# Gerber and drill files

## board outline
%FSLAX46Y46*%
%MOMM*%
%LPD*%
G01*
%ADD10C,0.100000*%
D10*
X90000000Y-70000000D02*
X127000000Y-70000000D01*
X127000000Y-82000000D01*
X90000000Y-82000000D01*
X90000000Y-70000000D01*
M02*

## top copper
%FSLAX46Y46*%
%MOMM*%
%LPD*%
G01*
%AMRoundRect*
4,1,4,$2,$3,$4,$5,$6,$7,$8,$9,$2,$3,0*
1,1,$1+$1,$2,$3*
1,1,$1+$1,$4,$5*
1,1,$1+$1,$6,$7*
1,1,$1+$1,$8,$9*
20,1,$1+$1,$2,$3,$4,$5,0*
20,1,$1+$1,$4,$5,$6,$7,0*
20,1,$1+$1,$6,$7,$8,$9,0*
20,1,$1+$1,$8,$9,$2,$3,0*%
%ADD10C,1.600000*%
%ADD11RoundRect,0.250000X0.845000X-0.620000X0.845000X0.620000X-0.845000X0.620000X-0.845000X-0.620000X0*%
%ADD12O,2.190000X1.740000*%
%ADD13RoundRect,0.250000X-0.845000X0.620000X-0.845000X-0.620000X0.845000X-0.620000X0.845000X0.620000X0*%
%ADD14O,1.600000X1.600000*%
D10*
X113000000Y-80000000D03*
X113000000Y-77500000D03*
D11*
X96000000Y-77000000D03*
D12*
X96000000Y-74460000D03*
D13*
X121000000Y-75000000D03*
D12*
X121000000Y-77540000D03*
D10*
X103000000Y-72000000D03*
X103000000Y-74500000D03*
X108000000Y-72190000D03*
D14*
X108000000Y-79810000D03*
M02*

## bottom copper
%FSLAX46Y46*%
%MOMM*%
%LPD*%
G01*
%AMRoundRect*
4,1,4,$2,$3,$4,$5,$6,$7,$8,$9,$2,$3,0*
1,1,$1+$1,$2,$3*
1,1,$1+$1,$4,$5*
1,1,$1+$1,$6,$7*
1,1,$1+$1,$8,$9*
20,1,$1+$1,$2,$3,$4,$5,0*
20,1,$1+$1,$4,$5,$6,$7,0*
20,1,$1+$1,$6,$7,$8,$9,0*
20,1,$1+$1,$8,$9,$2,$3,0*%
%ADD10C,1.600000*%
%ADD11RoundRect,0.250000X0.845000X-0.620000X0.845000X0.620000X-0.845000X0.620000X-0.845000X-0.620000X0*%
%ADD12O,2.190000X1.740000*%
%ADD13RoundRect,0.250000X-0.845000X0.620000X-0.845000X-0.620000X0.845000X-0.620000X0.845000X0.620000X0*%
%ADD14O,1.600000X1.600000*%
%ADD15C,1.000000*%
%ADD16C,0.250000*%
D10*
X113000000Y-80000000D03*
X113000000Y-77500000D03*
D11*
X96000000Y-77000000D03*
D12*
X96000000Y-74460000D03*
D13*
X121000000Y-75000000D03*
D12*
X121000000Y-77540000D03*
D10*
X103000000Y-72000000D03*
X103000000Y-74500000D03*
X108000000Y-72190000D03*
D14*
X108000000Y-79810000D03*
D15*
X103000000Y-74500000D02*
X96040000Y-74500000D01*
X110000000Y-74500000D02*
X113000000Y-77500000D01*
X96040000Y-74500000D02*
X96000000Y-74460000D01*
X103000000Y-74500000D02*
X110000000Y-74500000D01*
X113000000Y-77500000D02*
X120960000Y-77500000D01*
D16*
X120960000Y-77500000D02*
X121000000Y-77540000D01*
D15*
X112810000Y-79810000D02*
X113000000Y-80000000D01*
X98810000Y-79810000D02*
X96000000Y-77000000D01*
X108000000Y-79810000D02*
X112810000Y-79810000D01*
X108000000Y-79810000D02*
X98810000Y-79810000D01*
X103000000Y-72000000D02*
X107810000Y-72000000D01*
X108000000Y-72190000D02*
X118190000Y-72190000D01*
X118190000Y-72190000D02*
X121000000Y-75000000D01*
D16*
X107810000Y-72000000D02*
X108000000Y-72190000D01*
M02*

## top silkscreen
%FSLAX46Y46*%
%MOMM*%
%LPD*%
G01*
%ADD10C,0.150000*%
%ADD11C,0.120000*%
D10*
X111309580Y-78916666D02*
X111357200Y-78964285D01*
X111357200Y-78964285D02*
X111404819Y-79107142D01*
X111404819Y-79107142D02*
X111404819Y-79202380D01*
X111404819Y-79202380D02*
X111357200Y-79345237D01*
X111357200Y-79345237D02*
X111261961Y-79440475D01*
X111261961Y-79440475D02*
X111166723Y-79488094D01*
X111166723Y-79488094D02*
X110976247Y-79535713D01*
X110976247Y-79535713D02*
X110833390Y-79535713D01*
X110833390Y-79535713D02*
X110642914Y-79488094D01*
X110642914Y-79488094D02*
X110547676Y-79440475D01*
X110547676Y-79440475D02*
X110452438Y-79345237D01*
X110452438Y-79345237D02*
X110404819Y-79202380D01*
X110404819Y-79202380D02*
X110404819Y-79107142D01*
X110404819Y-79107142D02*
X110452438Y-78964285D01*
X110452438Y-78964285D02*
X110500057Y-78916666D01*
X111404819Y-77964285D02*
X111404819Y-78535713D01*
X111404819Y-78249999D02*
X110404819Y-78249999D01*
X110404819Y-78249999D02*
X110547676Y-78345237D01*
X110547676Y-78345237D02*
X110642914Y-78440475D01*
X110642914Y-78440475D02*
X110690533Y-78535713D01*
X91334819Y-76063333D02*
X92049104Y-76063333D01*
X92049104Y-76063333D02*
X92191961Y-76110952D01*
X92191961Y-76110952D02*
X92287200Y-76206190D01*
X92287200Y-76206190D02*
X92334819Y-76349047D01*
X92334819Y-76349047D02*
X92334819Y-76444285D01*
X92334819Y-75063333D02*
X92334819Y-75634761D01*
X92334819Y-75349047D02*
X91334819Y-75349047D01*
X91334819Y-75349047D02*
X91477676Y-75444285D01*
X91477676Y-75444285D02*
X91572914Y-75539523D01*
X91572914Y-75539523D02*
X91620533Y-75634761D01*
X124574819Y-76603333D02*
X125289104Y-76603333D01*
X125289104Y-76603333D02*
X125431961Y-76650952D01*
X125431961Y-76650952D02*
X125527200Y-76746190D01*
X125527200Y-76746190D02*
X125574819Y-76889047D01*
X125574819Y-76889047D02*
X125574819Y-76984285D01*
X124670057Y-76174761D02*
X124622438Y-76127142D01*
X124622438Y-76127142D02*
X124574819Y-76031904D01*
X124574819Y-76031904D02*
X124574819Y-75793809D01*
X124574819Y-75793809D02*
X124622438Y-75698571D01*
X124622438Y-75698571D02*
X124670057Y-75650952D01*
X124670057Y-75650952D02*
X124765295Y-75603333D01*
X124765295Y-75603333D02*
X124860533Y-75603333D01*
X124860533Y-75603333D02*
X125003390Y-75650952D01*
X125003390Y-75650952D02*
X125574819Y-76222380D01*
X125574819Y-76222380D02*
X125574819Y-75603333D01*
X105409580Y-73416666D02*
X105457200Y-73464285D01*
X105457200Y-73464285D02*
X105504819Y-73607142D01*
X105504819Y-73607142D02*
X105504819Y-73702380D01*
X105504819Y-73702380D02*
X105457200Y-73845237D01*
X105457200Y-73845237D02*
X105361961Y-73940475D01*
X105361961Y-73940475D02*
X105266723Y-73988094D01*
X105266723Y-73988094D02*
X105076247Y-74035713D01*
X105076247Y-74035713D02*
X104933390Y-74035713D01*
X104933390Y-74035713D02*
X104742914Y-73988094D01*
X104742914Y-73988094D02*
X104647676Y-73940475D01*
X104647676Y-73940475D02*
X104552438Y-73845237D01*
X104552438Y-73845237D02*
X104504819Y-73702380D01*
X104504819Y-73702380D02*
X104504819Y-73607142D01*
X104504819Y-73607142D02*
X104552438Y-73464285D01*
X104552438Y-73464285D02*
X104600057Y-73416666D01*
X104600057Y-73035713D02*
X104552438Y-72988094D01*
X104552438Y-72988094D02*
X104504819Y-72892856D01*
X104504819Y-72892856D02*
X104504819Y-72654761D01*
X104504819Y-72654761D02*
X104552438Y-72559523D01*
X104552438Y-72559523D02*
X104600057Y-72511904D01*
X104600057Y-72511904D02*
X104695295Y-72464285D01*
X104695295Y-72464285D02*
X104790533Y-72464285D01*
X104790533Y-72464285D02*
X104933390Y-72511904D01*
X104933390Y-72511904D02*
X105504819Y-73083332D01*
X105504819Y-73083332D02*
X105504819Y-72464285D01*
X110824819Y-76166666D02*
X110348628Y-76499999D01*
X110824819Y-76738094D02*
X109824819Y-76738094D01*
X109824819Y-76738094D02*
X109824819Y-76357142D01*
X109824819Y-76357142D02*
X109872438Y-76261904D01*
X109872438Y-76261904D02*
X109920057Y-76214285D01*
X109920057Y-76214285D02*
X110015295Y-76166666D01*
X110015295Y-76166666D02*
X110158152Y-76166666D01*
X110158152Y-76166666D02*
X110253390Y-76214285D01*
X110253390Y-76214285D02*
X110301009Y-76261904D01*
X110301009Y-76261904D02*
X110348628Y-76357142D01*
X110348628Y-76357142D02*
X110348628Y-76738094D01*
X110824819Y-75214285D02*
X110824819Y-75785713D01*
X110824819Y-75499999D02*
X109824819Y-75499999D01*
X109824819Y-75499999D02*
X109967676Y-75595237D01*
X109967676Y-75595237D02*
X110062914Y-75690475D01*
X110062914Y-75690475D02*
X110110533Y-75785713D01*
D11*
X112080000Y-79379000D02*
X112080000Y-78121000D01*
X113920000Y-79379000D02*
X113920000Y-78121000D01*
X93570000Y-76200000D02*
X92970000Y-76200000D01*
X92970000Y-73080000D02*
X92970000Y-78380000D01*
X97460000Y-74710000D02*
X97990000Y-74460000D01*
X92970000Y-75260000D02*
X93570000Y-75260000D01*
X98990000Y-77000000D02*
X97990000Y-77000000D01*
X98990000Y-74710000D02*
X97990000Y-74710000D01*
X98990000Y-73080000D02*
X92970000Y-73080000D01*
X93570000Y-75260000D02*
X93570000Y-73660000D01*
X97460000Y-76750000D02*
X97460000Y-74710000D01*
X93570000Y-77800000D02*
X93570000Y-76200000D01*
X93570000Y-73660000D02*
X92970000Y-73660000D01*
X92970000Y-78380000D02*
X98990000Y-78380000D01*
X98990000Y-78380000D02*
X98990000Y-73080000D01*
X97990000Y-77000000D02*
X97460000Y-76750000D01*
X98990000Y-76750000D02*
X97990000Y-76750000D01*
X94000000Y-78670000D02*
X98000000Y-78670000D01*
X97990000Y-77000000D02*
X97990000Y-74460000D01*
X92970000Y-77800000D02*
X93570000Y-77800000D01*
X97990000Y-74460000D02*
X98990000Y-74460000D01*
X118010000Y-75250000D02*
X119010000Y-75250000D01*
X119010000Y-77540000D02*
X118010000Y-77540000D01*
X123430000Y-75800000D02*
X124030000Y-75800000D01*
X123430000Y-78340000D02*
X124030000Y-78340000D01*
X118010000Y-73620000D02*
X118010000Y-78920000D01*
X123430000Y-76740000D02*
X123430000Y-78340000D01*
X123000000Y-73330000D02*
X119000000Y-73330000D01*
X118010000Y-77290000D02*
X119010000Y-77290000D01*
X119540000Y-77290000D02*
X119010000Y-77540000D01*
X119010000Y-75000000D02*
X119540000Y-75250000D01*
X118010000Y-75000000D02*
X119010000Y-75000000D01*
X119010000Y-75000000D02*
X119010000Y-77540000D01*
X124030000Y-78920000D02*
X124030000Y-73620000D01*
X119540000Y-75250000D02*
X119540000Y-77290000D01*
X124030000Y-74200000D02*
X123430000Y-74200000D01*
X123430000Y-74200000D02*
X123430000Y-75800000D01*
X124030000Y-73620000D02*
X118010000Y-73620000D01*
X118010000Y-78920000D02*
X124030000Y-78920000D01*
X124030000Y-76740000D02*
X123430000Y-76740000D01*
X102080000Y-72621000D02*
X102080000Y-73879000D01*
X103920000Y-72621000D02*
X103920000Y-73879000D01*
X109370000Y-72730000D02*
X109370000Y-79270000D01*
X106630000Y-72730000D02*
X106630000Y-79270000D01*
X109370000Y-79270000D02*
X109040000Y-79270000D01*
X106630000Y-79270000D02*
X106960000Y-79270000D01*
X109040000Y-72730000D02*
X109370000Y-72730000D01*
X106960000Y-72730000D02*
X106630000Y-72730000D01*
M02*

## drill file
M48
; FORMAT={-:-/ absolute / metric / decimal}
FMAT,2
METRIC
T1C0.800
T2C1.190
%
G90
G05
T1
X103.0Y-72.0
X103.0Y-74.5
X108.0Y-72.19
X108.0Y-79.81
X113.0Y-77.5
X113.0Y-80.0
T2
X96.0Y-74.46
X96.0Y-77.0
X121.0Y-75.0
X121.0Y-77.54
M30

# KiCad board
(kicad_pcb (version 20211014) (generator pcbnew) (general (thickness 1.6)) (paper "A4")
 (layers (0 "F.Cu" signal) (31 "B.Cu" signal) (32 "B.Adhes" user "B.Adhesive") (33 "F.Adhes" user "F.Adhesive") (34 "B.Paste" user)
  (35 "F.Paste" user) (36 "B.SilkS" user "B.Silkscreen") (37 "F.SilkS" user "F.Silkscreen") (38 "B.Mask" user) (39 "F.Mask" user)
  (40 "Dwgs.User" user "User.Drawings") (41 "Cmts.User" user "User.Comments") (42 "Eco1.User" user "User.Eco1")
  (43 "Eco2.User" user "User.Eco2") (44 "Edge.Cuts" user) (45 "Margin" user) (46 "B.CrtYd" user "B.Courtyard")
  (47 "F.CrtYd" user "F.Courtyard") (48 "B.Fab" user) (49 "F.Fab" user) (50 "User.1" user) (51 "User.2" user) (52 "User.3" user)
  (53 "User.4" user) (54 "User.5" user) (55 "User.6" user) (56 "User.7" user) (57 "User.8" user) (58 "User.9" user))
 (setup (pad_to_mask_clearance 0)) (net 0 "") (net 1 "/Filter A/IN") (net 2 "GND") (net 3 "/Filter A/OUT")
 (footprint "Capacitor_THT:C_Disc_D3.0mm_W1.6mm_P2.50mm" (layer "F.Cu") (at 113 80 90)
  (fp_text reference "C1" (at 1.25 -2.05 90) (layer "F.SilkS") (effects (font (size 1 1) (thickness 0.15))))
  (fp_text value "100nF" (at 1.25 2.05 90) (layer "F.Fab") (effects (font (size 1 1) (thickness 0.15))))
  (fp_line (start 0.621 -0.92) (end 1.879 -0.92) (layer "F.SilkS") (width 0.12))
  (fp_line (start 0.621 0.92) (end 1.879 0.92) (layer "F.SilkS") (width 0.12))
  (pad "1" thru_hole circle (at 0 0 90) (size 1.6 1.6) (drill 0.8) (layers *.Cu *.Mask) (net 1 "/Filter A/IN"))
  (pad "2" thru_hole circle (at 2.5 0 90) (size 1.6 1.6) (drill 0.8) (layers *.Cu *.Mask) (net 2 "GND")))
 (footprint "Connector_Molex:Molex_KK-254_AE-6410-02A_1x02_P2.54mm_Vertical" (layer "F.Cu") (at 96 77 90)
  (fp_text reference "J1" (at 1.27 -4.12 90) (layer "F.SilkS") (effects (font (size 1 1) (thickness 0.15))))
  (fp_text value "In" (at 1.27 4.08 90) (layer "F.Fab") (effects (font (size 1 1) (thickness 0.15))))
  (fp_line (start 0.8 -2.43) (end 0.8 -3.03) (layer "F.SilkS") (width 0.12))
  (fp_line (start 3.92 -3.03) (end -1.38 -3.03) (layer "F.SilkS") (width 0.12))
  (fp_line (start 2.29 1.46) (end 2.54 1.99) (layer "F.SilkS") (width 0.12))
  (fp_line (start 1.74 -3.03) (end 1.74 -2.43) (layer "F.SilkS") (width 0.12))
  (fp_line (start 0 2.99) (end 0 1.99) (layer "F.SilkS") (width 0.12))
  (fp_line (start 2.29 2.99) (end 2.29 1.99) (layer "F.SilkS") (width 0.12))
  (fp_line (start 3.92 2.99) (end 3.92 -3.03) (layer "F.SilkS") (width 0.12))
  (fp_line (start 1.74 -2.43) (end 3.34 -2.43) (layer "F.SilkS") (width 0.12))
  (fp_line (start 0.25 1.46) (end 2.29 1.46) (layer "F.SilkS") (width 0.12))
  (fp_line (start -0.8 -2.43) (end 0.8 -2.43) (layer "F.SilkS") (width 0.12))
  (fp_line (start 3.34 -2.43) (end 3.34 -3.03) (layer "F.SilkS") (width 0.12))
  (fp_line (start -1.38 -3.03) (end -1.38 2.99) (layer "F.SilkS") (width 0.12))
  (fp_line (start -1.38 2.99) (end 3.92 2.99) (layer "F.SilkS") (width 0.12))
  (fp_line (start 0 1.99) (end 0.25 1.46) (layer "F.SilkS") (width 0.12))
  (fp_line (start 0.25 2.99) (end 0.25 1.99) (layer "F.SilkS") (width 0.12))
  (fp_line (start -1.67 -2) (end -1.67 2) (layer "F.SilkS") (width 0.12))
  (fp_line (start 0 1.99) (end 2.54 1.99) (layer "F.SilkS") (width 0.12))
  (fp_line (start -0.8 -3.03) (end -0.8 -2.43) (layer "F.SilkS") (width 0.12))
  (fp_line (start 2.54 1.99) (end 2.54 2.99) (layer "F.SilkS") (width 0.12))
  (pad "1" thru_hole roundrect (at 0 0 90) (size 1.74 2.19) (drill 1.19) (layers *.Cu *.Mask) (roundrect_rratio 0.143678)
   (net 1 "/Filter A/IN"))
  (pad "2" thru_hole oval (at 2.54 0 90) (size 1.74 2.19) (drill 1.19) (layers *.Cu *.Mask) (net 2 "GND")))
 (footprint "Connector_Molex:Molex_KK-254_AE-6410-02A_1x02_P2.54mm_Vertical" (layer "F.Cu") (at 121 75 -90)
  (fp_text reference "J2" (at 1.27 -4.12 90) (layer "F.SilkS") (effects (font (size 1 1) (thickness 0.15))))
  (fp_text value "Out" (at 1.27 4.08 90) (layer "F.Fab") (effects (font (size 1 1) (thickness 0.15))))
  (fp_line (start 0.25 2.99) (end 0.25 1.99) (layer "F.SilkS") (width 0.12))
  (fp_line (start 2.54 1.99) (end 2.54 2.99) (layer "F.SilkS") (width 0.12))
  (fp_line (start 0.8 -2.43) (end 0.8 -3.03) (layer "F.SilkS") (width 0.12))
  (fp_line (start 3.34 -2.43) (end 3.34 -3.03) (layer "F.SilkS") (width 0.12))
  (fp_line (start -1.38 2.99) (end 3.92 2.99) (layer "F.SilkS") (width 0.12))
  (fp_line (start 1.74 -2.43) (end 3.34 -2.43) (layer "F.SilkS") (width 0.12))
  (fp_line (start -1.67 -2) (end -1.67 2) (layer "F.SilkS") (width 0.12))
  (fp_line (start 2.29 2.99) (end 2.29 1.99) (layer "F.SilkS") (width 0.12))
  (fp_line (start 2.29 1.46) (end 2.54 1.99) (layer "F.SilkS") (width 0.12))
  (fp_line (start 0 1.99) (end 0.25 1.46) (layer "F.SilkS") (width 0.12))
  (fp_line (start 0 2.99) (end 0 1.99) (layer "F.SilkS") (width 0.12))
  (fp_line (start 0 1.99) (end 2.54 1.99) (layer "F.SilkS") (width 0.12))
  (fp_line (start 3.92 -3.03) (end -1.38 -3.03) (layer "F.SilkS") (width 0.12))
  (fp_line (start 0.25 1.46) (end 2.29 1.46) (layer "F.SilkS") (width 0.12))
  (fp_line (start -0.8 -3.03) (end -0.8 -2.43) (layer "F.SilkS") (width 0.12))
  (fp_line (start -0.8 -2.43) (end 0.8 -2.43) (layer "F.SilkS") (width 0.12))
  (fp_line (start -1.38 -3.03) (end -1.38 2.99) (layer "F.SilkS") (width 0.12))
  (fp_line (start 3.92 2.99) (end 3.92 -3.03) (layer "F.SilkS") (width 0.12))
  (fp_line (start 1.74 -3.03) (end 1.74 -2.43) (layer "F.SilkS") (width 0.12))
  (pad "1" thru_hole roundrect (at 0 0 270) (size 1.74 2.19) (drill 1.19) (layers *.Cu *.Mask) (roundrect_rratio 0.143678)
   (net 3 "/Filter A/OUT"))
  (pad "2" thru_hole oval (at 2.54 0 270) (size 1.74 2.19) (drill 1.19) (layers *.Cu *.Mask) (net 2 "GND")))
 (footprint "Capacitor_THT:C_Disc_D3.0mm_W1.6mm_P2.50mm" (layer "F.Cu") (at 103 72 -90)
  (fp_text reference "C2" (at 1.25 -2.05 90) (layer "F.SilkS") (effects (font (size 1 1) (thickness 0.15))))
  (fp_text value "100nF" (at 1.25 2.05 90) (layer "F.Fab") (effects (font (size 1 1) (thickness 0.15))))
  (fp_line (start 0.621 0.92) (end 1.879 0.92) (layer "F.SilkS") (width 0.12))
  (fp_line (start 0.621 -0.92) (end 1.879 -0.92) (layer "F.SilkS") (width 0.12))
  (pad "1" thru_hole circle (at 0 0 270) (size 1.6 1.6) (drill 0.8) (layers *.Cu *.Mask) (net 3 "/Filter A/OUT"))
  (pad "2" thru_hole circle (at 2.5 0 270) (size 1.6 1.6) (drill 0.8) (layers *.Cu *.Mask) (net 2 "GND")))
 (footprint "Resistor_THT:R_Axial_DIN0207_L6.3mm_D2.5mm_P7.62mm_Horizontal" (layer "F.Cu") (at 108 72.19 -90)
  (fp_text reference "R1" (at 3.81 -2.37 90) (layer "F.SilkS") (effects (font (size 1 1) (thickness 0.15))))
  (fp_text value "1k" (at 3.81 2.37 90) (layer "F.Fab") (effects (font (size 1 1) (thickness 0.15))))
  (fp_line (start 0.54 -1.37) (end 7.08 -1.37) (layer "F.SilkS") (width 0.12))
  (fp_line (start 0.54 1.37) (end 7.08 1.37) (layer "F.SilkS") (width 0.12))
  (fp_line (start 7.08 -1.37) (end 7.08 -1.04) (layer "F.SilkS") (width 0.12))
  (fp_line (start 7.08 1.37) (end 7.08 1.04) (layer "F.SilkS") (width 0.12))
  (fp_line (start 0.54 -1.04) (end 0.54 -1.37) (layer "F.SilkS") (width 0.12))
  (fp_line (start 0.54 1.04) (end 0.54 1.37) (layer "F.SilkS") (width 0.12))
  (pad "1" thru_hole circle (at 0 0 270) (size 1.6 1.6) (drill 0.8) (layers *.Cu *.Mask) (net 3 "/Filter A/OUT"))
  (pad "2" thru_hole oval (at 7.62 0 270) (size 1.6 1.6) (drill 0.8) (layers *.Cu *.Mask) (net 1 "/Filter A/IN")))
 (gr_rect (start 90 70) (end 127 82) (layer "Edge.Cuts") (width 0.1) (fill none))
 (segment (start 103 74.5) (end 96.04 74.5) (width 1) (layer "B.Cu") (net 2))
 (segment (start 110 74.5) (end 113 77.5) (width 1) (layer "B.Cu") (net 2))
 (segment (start 96.04 74.5) (end 96 74.46) (width 1) (layer "B.Cu") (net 2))
 (segment (start 103 74.5) (end 110 74.5) (width 1) (layer "B.Cu") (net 2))
 (segment (start 113 77.5) (end 120.96 77.5) (width 1) (layer "B.Cu") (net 2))
 (segment (start 120.96 77.5) (end 121 77.54) (width 0.25) (layer "B.Cu") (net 2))
 (segment (start 112.81 79.81) (end 113 80) (width 1) (layer "B.Cu") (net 1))
 (segment (start 98.81 79.81) (end 96 77) (width 1) (layer "B.Cu") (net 1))
 (segment (start 108 79.81) (end 112.81 79.81) (width 1) (layer "B.Cu") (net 1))
 (segment (start 108 79.81) (end 98.81 79.81) (width 1) (layer "B.Cu") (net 1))
 (segment (start 103 72) (end 107.81 72) (width 1) (layer "B.Cu") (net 3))
 (segment (start 108 72.19) (end 118.19 72.19) (width 1) (layer "B.Cu") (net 3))
 (segment (start 118.19 72.19) (end 121 75) (width 1) (layer "B.Cu") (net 3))
 (segment (start 107.81 72) (end 108 72.19) (width 0.25) (layer "B.Cu") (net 3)))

